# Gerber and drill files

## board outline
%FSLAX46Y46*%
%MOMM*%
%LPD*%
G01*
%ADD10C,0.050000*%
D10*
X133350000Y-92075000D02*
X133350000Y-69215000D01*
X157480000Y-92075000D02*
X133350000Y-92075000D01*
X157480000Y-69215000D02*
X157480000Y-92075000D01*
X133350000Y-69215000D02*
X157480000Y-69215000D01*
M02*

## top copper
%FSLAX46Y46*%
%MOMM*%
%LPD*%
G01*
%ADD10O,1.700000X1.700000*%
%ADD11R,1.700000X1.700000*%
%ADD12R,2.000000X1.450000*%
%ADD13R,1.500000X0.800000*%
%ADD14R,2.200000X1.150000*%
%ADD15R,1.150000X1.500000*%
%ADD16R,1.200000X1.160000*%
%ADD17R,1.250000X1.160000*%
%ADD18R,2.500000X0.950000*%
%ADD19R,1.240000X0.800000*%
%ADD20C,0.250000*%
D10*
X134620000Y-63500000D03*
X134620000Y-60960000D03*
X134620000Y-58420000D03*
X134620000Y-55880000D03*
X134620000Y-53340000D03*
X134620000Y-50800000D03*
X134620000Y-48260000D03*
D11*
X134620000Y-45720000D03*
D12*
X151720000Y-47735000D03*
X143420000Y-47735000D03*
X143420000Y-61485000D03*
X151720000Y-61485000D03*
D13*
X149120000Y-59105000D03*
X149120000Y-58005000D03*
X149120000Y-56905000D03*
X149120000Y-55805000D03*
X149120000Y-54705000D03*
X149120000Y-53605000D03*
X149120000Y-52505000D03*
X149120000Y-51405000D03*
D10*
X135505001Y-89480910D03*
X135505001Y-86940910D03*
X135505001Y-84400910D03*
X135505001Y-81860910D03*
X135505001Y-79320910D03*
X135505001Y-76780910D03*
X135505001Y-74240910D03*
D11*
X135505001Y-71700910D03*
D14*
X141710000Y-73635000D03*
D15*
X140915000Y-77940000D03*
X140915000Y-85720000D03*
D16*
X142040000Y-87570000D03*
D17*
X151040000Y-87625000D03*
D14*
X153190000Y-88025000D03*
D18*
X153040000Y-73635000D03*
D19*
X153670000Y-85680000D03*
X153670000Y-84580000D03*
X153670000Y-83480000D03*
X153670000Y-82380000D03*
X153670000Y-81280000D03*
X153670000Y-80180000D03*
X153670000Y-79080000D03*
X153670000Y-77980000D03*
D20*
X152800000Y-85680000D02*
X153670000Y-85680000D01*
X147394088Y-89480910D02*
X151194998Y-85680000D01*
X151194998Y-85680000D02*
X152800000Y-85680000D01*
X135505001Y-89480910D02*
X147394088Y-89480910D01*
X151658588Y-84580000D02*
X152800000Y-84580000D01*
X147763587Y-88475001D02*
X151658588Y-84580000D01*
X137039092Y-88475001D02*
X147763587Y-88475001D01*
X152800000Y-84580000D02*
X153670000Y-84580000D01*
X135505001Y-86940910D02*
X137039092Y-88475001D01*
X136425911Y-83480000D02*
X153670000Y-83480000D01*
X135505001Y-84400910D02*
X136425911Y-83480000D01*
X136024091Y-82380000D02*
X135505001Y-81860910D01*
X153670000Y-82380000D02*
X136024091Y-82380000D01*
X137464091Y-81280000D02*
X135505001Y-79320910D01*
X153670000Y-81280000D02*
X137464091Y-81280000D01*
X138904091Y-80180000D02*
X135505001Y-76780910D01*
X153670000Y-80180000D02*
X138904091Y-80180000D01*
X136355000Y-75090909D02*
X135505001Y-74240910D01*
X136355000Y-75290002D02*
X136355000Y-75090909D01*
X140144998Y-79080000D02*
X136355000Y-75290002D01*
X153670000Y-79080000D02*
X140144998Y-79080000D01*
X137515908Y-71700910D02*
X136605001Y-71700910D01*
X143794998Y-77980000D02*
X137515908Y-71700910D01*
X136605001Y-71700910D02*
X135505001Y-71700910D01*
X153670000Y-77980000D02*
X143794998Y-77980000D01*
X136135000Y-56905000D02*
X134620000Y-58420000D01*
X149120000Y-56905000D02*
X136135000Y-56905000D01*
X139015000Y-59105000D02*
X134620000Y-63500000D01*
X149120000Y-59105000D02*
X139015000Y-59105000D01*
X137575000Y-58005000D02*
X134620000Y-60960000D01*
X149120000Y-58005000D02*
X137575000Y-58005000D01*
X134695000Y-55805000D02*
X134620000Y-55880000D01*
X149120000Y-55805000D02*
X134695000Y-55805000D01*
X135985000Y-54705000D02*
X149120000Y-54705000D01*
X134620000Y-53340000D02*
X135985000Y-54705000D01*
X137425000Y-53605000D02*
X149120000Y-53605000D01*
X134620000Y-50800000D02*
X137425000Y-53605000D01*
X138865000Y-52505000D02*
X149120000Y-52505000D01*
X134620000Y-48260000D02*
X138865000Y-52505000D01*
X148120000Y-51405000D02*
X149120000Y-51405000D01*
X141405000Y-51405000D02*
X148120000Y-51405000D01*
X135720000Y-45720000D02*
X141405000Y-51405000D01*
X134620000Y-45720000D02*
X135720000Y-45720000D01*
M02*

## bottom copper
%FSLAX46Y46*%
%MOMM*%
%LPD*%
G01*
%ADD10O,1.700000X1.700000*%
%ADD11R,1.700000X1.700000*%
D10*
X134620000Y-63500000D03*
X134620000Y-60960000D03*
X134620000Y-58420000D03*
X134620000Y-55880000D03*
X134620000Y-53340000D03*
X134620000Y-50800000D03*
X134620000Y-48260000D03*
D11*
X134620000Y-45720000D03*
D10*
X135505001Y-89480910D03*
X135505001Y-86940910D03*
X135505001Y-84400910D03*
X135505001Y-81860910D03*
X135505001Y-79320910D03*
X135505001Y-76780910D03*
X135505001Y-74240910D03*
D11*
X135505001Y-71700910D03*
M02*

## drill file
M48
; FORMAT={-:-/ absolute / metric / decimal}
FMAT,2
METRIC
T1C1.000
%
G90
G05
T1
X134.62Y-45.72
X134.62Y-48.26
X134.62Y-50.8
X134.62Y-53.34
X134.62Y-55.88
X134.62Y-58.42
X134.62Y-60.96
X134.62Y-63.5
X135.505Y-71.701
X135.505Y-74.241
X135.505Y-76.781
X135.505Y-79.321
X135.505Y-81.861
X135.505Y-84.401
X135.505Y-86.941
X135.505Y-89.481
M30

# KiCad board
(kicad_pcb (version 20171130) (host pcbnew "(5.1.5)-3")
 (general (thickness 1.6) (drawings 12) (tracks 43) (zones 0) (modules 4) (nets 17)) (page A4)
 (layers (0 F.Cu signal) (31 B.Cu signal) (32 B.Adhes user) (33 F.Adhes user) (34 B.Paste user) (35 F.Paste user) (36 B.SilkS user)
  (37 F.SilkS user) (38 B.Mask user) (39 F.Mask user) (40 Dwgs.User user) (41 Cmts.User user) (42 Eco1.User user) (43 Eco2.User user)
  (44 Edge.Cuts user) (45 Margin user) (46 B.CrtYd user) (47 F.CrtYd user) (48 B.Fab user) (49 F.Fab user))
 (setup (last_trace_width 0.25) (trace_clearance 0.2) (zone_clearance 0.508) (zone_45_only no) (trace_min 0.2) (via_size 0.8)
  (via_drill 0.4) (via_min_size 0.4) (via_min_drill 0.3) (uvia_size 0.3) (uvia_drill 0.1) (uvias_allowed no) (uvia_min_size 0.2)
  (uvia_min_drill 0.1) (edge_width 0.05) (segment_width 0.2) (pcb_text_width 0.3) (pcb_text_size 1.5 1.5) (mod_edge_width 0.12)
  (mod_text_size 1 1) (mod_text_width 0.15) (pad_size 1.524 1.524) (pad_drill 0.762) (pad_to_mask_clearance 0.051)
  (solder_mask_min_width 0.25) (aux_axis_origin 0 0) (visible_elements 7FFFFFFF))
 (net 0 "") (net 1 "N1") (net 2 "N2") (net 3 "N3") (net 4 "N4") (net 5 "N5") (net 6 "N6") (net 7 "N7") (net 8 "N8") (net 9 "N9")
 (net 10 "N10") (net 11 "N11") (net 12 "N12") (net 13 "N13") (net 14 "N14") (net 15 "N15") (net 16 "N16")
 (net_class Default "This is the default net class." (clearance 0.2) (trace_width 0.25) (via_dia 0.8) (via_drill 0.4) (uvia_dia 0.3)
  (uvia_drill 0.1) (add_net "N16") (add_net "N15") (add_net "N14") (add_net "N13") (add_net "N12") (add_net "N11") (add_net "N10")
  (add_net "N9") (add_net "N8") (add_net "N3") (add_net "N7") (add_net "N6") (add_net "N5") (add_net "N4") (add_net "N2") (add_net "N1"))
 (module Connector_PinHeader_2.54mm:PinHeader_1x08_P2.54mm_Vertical (layer F.Cu) (at 134.62 45.72)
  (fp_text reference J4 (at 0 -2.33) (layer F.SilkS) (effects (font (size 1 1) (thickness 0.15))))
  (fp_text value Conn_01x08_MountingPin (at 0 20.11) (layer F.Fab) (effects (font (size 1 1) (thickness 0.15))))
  (pad 8 thru_hole oval (at 0 17.78) (size 1.7 1.7) (drill 1) (layers *.Cu *.Mask) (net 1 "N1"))
  (pad 7 thru_hole oval (at 0 15.24) (size 1.7 1.7) (drill 1) (layers *.Cu *.Mask) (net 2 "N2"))
  (pad 6 thru_hole oval (at 0 12.7) (size 1.7 1.7) (drill 1) (layers *.Cu *.Mask) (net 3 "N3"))
  (pad 5 thru_hole oval (at 0 10.16) (size 1.7 1.7) (drill 1) (layers *.Cu *.Mask) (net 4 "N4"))
  (pad 4 thru_hole oval (at 0 7.62) (size 1.7 1.7) (drill 1) (layers *.Cu *.Mask) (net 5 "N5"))
  (pad 3 thru_hole oval (at 0 5.08) (size 1.7 1.7) (drill 1) (layers *.Cu *.Mask) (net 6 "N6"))
  (pad 2 thru_hole oval (at 0 2.54) (size 1.7 1.7) (drill 1) (layers *.Cu *.Mask) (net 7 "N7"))
  (pad 1 thru_hole rect (at 0 0) (size 1.7 1.7) (drill 1) (layers *.Cu *.Mask) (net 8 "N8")))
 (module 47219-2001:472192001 (layer F.Cu) (at 147.32 54.61 90)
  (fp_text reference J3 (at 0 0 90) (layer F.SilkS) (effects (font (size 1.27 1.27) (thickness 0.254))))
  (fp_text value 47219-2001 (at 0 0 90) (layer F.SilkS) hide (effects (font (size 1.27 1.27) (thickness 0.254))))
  (pad 12 smd rect (at 6.875 4.4 90) (size 1.45 2) (layers F.Cu F.Paste F.Mask) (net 3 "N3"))
  (pad 11 smd rect (at 6.875 -3.9 90) (size 1.45 2) (layers F.Cu F.Paste F.Mask) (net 3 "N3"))
  (pad 10 smd rect (at -6.875 -3.9 90) (size 1.45 2) (layers F.Cu F.Paste F.Mask) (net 3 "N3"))
  (pad 9 smd rect (at -6.875 4.4 90) (size 1.45 2) (layers F.Cu F.Paste F.Mask) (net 3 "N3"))
  (pad 8 smd rect (at -4.495 1.8 90) (size 0.8 1.5) (layers F.Cu F.Paste F.Mask) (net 1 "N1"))
  (pad 7 smd rect (at -3.395 1.8 90) (size 0.8 1.5) (layers F.Cu F.Paste F.Mask) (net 2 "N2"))
  (pad 6 smd rect (at -2.295 1.8 90) (size 0.8 1.5) (layers F.Cu F.Paste F.Mask) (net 3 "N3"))
  (pad 5 smd rect (at -1.195 1.8 90) (size 0.8 1.5) (layers F.Cu F.Paste F.Mask) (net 4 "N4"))
  (pad 4 smd rect (at -0.095 1.8 90) (size 0.8 1.5) (layers F.Cu F.Paste F.Mask) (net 5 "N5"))
  (pad 3 smd rect (at 1.005 1.8 90) (size 0.8 1.5) (layers F.Cu F.Paste F.Mask) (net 6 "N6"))
  (pad 2 smd rect (at 2.105 1.8 90) (size 0.8 1.5) (layers F.Cu F.Paste F.Mask) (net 7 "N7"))
  (pad 1 smd rect (at 3.205 1.8 90) (size 0.8 1.5) (layers F.Cu F.Paste F.Mask) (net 8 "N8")))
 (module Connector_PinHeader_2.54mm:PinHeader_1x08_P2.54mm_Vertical (layer B.Cu) (at 135.505001 71.70091 180)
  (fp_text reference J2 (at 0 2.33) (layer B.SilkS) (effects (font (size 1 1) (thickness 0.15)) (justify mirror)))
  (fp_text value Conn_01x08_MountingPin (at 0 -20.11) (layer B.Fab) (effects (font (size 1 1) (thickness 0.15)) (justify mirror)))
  (pad 8 thru_hole oval (at 0 -17.78 180) (size 1.7 1.7) (drill 1) (layers *.Cu *.Mask) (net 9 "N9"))
  (pad 7 thru_hole oval (at 0 -15.24 180) (size 1.7 1.7) (drill 1) (layers *.Cu *.Mask) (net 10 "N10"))
  (pad 6 thru_hole oval (at 0 -12.7 180) (size 1.7 1.7) (drill 1) (layers *.Cu *.Mask) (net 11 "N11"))
  (pad 5 thru_hole oval (at 0 -10.16 180) (size 1.7 1.7) (drill 1) (layers *.Cu *.Mask) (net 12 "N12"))
  (pad 4 thru_hole oval (at 0 -7.62 180) (size 1.7 1.7) (drill 1) (layers *.Cu *.Mask) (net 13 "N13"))
  (pad 3 thru_hole oval (at 0 -5.08 180) (size 1.7 1.7) (drill 1) (layers *.Cu *.Mask) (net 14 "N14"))
  (pad 2 thru_hole oval (at 0 -2.54 180) (size 1.7 1.7) (drill 1) (layers *.Cu *.Mask) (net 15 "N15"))
  (pad 1 thru_hole rect (at 0 0 180) (size 1.7 1.7) (drill 1) (layers *.Cu *.Mask) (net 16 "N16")))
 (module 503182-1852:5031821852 (layer F.Cu) (at 153.04 80.83 270)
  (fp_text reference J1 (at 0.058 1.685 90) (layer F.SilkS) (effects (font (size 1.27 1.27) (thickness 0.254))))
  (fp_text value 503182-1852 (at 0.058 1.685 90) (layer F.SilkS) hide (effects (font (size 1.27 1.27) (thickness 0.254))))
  (pad 15 smd rect (at -7.195 11.33 270) (size 1.15 2.2) (layers F.Cu F.Paste F.Mask))
  (pad 14 smd rect (at -2.89 12.125) (size 1.15 1.5) (layers F.Cu F.Paste F.Mask))
  (pad 13 smd rect (at 4.89 12.125) (size 1.15 1.5) (layers F.Cu F.Paste F.Mask))
  (pad 12 smd rect (at 6.74 11 270) (size 1.16 1.2) (layers F.Cu F.Paste F.Mask))
  (pad 11 smd rect (at 6.795 2 270) (size 1.16 1.25) (layers F.Cu F.Paste F.Mask))
  (pad 10 smd rect (at 7.195 -0.15 270) (size 1.15 2.2) (layers F.Cu F.Paste F.Mask))
  (pad 9 smd rect (at -7.195 0 270) (size 0.95 2.5) (layers F.Cu F.Paste F.Mask))
  (pad 8 smd rect (at 4.85 -0.63 270) (size 0.8 1.24) (layers F.Cu F.Paste F.Mask) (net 9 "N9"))
  (pad 7 smd rect (at 3.75 -0.63 270) (size 0.8 1.24) (layers F.Cu F.Paste F.Mask) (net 10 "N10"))
  (pad 6 smd rect (at 2.65 -0.63 270) (size 0.8 1.24) (layers F.Cu F.Paste F.Mask) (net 11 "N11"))
  (pad 5 smd rect (at 1.55 -0.63 270) (size 0.8 1.24) (layers F.Cu F.Paste F.Mask) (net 12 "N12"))
  (pad 4 smd rect (at 0.45 -0.63 270) (size 0.8 1.24) (layers F.Cu F.Paste F.Mask) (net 13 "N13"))
  (pad 3 smd rect (at -0.65 -0.63 270) (size 0.8 1.24) (layers F.Cu F.Paste F.Mask) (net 14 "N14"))
  (pad 2 smd rect (at -1.75 -0.63 270) (size 0.8 1.24) (layers F.Cu F.Paste F.Mask) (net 15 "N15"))
  (pad 1 smd rect (at -2.85 -0.63 270) (size 0.8 1.24) (layers F.Cu F.Paste F.Mask) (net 16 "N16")))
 (gr_line (start 133.35 92.075) (end 133.35 69.215) (layer Edge.Cuts) (width 0.05))
 (gr_line (start 157.48 92.075) (end 133.35 92.075) (layer Edge.Cuts) (width 0.05))
 (gr_line (start 157.48 69.215) (end 157.48 92.075) (layer Edge.Cuts) (width 0.05))
 (gr_line (start 133.35 69.215) (end 157.48 69.215) (layer Edge.Cuts) (width 0.05))
 (segment (start 152.8 85.68) (end 153.67 85.68) (width 0.25) (layer F.Cu) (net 9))
 (segment (start 147.394088 89.48091) (end 151.194998 85.68) (width 0.25) (layer F.Cu) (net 9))
 (segment (start 151.194998 85.68) (end 152.8 85.68) (width 0.25) (layer F.Cu) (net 9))
 (segment (start 135.505001 89.48091) (end 147.394088 89.48091) (width 0.25) (layer F.Cu) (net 9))
 (segment (start 151.658588 84.58) (end 152.8 84.58) (width 0.25) (layer F.Cu) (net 10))
 (segment (start 147.763587 88.475001) (end 151.658588 84.58) (width 0.25) (layer F.Cu) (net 10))
 (segment (start 137.039092 88.475001) (end 147.763587 88.475001) (width 0.25) (layer F.Cu) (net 10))
 (segment (start 152.8 84.58) (end 153.67 84.58) (width 0.25) (layer F.Cu) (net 10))
 (segment (start 135.505001 86.94091) (end 137.039092 88.475001) (width 0.25) (layer F.Cu) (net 10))
 (segment (start 136.425911 83.48) (end 153.67 83.48) (width 0.25) (layer F.Cu) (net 11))
 (segment (start 135.505001 84.40091) (end 136.425911 83.48) (width 0.25) (layer F.Cu) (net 11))
 (segment (start 136.024091 82.38) (end 135.505001 81.86091) (width 0.25) (layer F.Cu) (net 12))
 (segment (start 153.67 82.38) (end 136.024091 82.38) (width 0.25) (layer F.Cu) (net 12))
 (segment (start 137.464091 81.28) (end 135.505001 79.32091) (width 0.25) (layer F.Cu) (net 13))
 (segment (start 153.67 81.28) (end 137.464091 81.28) (width 0.25) (layer F.Cu) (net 13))
 (segment (start 138.904091 80.18) (end 135.505001 76.78091) (width 0.25) (layer F.Cu) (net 14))
 (segment (start 153.67 80.18) (end 138.904091 80.18) (width 0.25) (layer F.Cu) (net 14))
 (segment (start 136.355 75.090909) (end 135.505001 74.24091) (width 0.25) (layer F.Cu) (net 15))
 (segment (start 136.355 75.290002) (end 136.355 75.090909) (width 0.25) (layer F.Cu) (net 15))
 (segment (start 140.144998 79.08) (end 136.355 75.290002) (width 0.25) (layer F.Cu) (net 15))
 (segment (start 153.67 79.08) (end 140.144998 79.08) (width 0.25) (layer F.Cu) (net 15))
 (segment (start 137.515908 71.70091) (end 136.605001 71.70091) (width 0.25) (layer F.Cu) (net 16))
 (segment (start 143.794998 77.98) (end 137.515908 71.70091) (width 0.25) (layer F.Cu) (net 16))
 (segment (start 136.605001 71.70091) (end 135.505001 71.70091) (width 0.25) (layer F.Cu) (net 16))
 (segment (start 153.67 77.98) (end 143.794998 77.98) (width 0.25) (layer F.Cu) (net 16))
 (segment (start 136.135 56.905) (end 134.62 58.42) (width 0.25) (layer F.Cu) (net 3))
 (segment (start 149.12 56.905) (end 136.135 56.905) (width 0.25) (layer F.Cu) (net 3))
 (segment (start 139.015 59.105) (end 134.62 63.5) (width 0.25) (layer F.Cu) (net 1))
 (segment (start 149.12 59.105) (end 139.015 59.105) (width 0.25) (layer F.Cu) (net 1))
 (segment (start 137.575 58.005) (end 134.62 60.96) (width 0.25) (layer F.Cu) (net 2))
 (segment (start 149.12 58.005) (end 137.575 58.005) (width 0.25) (layer F.Cu) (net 2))
 (segment (start 134.695 55.805) (end 134.62 55.88) (width 0.25) (layer F.Cu) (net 4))
 (segment (start 149.12 55.805) (end 134.695 55.805) (width 0.25) (layer F.Cu) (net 4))
 (segment (start 135.985 54.705) (end 149.12 54.705) (width 0.25) (layer F.Cu) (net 5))
 (segment (start 134.62 53.34) (end 135.985 54.705) (width 0.25) (layer F.Cu) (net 5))
 (segment (start 137.425 53.605) (end 149.12 53.605) (width 0.25) (layer F.Cu) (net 6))
 (segment (start 134.62 50.8) (end 137.425 53.605) (width 0.25) (layer F.Cu) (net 6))
 (segment (start 138.865 52.505) (end 149.12 52.505) (width 0.25) (layer F.Cu) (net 7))
 (segment (start 134.62 48.26) (end 138.865 52.505) (width 0.25) (layer F.Cu) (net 7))
 (segment (start 148.12 51.405) (end 149.12 51.405) (width 0.25) (layer F.Cu) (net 8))
 (segment (start 141.405 51.405) (end 148.12 51.405) (width 0.25) (layer F.Cu) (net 8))
 (segment (start 135.72 45.72) (end 141.405 51.405) (width 0.25) (layer F.Cu) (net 8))
 (segment (start 134.62 45.72) (end 135.72 45.72) (width 0.25) (layer F.Cu) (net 8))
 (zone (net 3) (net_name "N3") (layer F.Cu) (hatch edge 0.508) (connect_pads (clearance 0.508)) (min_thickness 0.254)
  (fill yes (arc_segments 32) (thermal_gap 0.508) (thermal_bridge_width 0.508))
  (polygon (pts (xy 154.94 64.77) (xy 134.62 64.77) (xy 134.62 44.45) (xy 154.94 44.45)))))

